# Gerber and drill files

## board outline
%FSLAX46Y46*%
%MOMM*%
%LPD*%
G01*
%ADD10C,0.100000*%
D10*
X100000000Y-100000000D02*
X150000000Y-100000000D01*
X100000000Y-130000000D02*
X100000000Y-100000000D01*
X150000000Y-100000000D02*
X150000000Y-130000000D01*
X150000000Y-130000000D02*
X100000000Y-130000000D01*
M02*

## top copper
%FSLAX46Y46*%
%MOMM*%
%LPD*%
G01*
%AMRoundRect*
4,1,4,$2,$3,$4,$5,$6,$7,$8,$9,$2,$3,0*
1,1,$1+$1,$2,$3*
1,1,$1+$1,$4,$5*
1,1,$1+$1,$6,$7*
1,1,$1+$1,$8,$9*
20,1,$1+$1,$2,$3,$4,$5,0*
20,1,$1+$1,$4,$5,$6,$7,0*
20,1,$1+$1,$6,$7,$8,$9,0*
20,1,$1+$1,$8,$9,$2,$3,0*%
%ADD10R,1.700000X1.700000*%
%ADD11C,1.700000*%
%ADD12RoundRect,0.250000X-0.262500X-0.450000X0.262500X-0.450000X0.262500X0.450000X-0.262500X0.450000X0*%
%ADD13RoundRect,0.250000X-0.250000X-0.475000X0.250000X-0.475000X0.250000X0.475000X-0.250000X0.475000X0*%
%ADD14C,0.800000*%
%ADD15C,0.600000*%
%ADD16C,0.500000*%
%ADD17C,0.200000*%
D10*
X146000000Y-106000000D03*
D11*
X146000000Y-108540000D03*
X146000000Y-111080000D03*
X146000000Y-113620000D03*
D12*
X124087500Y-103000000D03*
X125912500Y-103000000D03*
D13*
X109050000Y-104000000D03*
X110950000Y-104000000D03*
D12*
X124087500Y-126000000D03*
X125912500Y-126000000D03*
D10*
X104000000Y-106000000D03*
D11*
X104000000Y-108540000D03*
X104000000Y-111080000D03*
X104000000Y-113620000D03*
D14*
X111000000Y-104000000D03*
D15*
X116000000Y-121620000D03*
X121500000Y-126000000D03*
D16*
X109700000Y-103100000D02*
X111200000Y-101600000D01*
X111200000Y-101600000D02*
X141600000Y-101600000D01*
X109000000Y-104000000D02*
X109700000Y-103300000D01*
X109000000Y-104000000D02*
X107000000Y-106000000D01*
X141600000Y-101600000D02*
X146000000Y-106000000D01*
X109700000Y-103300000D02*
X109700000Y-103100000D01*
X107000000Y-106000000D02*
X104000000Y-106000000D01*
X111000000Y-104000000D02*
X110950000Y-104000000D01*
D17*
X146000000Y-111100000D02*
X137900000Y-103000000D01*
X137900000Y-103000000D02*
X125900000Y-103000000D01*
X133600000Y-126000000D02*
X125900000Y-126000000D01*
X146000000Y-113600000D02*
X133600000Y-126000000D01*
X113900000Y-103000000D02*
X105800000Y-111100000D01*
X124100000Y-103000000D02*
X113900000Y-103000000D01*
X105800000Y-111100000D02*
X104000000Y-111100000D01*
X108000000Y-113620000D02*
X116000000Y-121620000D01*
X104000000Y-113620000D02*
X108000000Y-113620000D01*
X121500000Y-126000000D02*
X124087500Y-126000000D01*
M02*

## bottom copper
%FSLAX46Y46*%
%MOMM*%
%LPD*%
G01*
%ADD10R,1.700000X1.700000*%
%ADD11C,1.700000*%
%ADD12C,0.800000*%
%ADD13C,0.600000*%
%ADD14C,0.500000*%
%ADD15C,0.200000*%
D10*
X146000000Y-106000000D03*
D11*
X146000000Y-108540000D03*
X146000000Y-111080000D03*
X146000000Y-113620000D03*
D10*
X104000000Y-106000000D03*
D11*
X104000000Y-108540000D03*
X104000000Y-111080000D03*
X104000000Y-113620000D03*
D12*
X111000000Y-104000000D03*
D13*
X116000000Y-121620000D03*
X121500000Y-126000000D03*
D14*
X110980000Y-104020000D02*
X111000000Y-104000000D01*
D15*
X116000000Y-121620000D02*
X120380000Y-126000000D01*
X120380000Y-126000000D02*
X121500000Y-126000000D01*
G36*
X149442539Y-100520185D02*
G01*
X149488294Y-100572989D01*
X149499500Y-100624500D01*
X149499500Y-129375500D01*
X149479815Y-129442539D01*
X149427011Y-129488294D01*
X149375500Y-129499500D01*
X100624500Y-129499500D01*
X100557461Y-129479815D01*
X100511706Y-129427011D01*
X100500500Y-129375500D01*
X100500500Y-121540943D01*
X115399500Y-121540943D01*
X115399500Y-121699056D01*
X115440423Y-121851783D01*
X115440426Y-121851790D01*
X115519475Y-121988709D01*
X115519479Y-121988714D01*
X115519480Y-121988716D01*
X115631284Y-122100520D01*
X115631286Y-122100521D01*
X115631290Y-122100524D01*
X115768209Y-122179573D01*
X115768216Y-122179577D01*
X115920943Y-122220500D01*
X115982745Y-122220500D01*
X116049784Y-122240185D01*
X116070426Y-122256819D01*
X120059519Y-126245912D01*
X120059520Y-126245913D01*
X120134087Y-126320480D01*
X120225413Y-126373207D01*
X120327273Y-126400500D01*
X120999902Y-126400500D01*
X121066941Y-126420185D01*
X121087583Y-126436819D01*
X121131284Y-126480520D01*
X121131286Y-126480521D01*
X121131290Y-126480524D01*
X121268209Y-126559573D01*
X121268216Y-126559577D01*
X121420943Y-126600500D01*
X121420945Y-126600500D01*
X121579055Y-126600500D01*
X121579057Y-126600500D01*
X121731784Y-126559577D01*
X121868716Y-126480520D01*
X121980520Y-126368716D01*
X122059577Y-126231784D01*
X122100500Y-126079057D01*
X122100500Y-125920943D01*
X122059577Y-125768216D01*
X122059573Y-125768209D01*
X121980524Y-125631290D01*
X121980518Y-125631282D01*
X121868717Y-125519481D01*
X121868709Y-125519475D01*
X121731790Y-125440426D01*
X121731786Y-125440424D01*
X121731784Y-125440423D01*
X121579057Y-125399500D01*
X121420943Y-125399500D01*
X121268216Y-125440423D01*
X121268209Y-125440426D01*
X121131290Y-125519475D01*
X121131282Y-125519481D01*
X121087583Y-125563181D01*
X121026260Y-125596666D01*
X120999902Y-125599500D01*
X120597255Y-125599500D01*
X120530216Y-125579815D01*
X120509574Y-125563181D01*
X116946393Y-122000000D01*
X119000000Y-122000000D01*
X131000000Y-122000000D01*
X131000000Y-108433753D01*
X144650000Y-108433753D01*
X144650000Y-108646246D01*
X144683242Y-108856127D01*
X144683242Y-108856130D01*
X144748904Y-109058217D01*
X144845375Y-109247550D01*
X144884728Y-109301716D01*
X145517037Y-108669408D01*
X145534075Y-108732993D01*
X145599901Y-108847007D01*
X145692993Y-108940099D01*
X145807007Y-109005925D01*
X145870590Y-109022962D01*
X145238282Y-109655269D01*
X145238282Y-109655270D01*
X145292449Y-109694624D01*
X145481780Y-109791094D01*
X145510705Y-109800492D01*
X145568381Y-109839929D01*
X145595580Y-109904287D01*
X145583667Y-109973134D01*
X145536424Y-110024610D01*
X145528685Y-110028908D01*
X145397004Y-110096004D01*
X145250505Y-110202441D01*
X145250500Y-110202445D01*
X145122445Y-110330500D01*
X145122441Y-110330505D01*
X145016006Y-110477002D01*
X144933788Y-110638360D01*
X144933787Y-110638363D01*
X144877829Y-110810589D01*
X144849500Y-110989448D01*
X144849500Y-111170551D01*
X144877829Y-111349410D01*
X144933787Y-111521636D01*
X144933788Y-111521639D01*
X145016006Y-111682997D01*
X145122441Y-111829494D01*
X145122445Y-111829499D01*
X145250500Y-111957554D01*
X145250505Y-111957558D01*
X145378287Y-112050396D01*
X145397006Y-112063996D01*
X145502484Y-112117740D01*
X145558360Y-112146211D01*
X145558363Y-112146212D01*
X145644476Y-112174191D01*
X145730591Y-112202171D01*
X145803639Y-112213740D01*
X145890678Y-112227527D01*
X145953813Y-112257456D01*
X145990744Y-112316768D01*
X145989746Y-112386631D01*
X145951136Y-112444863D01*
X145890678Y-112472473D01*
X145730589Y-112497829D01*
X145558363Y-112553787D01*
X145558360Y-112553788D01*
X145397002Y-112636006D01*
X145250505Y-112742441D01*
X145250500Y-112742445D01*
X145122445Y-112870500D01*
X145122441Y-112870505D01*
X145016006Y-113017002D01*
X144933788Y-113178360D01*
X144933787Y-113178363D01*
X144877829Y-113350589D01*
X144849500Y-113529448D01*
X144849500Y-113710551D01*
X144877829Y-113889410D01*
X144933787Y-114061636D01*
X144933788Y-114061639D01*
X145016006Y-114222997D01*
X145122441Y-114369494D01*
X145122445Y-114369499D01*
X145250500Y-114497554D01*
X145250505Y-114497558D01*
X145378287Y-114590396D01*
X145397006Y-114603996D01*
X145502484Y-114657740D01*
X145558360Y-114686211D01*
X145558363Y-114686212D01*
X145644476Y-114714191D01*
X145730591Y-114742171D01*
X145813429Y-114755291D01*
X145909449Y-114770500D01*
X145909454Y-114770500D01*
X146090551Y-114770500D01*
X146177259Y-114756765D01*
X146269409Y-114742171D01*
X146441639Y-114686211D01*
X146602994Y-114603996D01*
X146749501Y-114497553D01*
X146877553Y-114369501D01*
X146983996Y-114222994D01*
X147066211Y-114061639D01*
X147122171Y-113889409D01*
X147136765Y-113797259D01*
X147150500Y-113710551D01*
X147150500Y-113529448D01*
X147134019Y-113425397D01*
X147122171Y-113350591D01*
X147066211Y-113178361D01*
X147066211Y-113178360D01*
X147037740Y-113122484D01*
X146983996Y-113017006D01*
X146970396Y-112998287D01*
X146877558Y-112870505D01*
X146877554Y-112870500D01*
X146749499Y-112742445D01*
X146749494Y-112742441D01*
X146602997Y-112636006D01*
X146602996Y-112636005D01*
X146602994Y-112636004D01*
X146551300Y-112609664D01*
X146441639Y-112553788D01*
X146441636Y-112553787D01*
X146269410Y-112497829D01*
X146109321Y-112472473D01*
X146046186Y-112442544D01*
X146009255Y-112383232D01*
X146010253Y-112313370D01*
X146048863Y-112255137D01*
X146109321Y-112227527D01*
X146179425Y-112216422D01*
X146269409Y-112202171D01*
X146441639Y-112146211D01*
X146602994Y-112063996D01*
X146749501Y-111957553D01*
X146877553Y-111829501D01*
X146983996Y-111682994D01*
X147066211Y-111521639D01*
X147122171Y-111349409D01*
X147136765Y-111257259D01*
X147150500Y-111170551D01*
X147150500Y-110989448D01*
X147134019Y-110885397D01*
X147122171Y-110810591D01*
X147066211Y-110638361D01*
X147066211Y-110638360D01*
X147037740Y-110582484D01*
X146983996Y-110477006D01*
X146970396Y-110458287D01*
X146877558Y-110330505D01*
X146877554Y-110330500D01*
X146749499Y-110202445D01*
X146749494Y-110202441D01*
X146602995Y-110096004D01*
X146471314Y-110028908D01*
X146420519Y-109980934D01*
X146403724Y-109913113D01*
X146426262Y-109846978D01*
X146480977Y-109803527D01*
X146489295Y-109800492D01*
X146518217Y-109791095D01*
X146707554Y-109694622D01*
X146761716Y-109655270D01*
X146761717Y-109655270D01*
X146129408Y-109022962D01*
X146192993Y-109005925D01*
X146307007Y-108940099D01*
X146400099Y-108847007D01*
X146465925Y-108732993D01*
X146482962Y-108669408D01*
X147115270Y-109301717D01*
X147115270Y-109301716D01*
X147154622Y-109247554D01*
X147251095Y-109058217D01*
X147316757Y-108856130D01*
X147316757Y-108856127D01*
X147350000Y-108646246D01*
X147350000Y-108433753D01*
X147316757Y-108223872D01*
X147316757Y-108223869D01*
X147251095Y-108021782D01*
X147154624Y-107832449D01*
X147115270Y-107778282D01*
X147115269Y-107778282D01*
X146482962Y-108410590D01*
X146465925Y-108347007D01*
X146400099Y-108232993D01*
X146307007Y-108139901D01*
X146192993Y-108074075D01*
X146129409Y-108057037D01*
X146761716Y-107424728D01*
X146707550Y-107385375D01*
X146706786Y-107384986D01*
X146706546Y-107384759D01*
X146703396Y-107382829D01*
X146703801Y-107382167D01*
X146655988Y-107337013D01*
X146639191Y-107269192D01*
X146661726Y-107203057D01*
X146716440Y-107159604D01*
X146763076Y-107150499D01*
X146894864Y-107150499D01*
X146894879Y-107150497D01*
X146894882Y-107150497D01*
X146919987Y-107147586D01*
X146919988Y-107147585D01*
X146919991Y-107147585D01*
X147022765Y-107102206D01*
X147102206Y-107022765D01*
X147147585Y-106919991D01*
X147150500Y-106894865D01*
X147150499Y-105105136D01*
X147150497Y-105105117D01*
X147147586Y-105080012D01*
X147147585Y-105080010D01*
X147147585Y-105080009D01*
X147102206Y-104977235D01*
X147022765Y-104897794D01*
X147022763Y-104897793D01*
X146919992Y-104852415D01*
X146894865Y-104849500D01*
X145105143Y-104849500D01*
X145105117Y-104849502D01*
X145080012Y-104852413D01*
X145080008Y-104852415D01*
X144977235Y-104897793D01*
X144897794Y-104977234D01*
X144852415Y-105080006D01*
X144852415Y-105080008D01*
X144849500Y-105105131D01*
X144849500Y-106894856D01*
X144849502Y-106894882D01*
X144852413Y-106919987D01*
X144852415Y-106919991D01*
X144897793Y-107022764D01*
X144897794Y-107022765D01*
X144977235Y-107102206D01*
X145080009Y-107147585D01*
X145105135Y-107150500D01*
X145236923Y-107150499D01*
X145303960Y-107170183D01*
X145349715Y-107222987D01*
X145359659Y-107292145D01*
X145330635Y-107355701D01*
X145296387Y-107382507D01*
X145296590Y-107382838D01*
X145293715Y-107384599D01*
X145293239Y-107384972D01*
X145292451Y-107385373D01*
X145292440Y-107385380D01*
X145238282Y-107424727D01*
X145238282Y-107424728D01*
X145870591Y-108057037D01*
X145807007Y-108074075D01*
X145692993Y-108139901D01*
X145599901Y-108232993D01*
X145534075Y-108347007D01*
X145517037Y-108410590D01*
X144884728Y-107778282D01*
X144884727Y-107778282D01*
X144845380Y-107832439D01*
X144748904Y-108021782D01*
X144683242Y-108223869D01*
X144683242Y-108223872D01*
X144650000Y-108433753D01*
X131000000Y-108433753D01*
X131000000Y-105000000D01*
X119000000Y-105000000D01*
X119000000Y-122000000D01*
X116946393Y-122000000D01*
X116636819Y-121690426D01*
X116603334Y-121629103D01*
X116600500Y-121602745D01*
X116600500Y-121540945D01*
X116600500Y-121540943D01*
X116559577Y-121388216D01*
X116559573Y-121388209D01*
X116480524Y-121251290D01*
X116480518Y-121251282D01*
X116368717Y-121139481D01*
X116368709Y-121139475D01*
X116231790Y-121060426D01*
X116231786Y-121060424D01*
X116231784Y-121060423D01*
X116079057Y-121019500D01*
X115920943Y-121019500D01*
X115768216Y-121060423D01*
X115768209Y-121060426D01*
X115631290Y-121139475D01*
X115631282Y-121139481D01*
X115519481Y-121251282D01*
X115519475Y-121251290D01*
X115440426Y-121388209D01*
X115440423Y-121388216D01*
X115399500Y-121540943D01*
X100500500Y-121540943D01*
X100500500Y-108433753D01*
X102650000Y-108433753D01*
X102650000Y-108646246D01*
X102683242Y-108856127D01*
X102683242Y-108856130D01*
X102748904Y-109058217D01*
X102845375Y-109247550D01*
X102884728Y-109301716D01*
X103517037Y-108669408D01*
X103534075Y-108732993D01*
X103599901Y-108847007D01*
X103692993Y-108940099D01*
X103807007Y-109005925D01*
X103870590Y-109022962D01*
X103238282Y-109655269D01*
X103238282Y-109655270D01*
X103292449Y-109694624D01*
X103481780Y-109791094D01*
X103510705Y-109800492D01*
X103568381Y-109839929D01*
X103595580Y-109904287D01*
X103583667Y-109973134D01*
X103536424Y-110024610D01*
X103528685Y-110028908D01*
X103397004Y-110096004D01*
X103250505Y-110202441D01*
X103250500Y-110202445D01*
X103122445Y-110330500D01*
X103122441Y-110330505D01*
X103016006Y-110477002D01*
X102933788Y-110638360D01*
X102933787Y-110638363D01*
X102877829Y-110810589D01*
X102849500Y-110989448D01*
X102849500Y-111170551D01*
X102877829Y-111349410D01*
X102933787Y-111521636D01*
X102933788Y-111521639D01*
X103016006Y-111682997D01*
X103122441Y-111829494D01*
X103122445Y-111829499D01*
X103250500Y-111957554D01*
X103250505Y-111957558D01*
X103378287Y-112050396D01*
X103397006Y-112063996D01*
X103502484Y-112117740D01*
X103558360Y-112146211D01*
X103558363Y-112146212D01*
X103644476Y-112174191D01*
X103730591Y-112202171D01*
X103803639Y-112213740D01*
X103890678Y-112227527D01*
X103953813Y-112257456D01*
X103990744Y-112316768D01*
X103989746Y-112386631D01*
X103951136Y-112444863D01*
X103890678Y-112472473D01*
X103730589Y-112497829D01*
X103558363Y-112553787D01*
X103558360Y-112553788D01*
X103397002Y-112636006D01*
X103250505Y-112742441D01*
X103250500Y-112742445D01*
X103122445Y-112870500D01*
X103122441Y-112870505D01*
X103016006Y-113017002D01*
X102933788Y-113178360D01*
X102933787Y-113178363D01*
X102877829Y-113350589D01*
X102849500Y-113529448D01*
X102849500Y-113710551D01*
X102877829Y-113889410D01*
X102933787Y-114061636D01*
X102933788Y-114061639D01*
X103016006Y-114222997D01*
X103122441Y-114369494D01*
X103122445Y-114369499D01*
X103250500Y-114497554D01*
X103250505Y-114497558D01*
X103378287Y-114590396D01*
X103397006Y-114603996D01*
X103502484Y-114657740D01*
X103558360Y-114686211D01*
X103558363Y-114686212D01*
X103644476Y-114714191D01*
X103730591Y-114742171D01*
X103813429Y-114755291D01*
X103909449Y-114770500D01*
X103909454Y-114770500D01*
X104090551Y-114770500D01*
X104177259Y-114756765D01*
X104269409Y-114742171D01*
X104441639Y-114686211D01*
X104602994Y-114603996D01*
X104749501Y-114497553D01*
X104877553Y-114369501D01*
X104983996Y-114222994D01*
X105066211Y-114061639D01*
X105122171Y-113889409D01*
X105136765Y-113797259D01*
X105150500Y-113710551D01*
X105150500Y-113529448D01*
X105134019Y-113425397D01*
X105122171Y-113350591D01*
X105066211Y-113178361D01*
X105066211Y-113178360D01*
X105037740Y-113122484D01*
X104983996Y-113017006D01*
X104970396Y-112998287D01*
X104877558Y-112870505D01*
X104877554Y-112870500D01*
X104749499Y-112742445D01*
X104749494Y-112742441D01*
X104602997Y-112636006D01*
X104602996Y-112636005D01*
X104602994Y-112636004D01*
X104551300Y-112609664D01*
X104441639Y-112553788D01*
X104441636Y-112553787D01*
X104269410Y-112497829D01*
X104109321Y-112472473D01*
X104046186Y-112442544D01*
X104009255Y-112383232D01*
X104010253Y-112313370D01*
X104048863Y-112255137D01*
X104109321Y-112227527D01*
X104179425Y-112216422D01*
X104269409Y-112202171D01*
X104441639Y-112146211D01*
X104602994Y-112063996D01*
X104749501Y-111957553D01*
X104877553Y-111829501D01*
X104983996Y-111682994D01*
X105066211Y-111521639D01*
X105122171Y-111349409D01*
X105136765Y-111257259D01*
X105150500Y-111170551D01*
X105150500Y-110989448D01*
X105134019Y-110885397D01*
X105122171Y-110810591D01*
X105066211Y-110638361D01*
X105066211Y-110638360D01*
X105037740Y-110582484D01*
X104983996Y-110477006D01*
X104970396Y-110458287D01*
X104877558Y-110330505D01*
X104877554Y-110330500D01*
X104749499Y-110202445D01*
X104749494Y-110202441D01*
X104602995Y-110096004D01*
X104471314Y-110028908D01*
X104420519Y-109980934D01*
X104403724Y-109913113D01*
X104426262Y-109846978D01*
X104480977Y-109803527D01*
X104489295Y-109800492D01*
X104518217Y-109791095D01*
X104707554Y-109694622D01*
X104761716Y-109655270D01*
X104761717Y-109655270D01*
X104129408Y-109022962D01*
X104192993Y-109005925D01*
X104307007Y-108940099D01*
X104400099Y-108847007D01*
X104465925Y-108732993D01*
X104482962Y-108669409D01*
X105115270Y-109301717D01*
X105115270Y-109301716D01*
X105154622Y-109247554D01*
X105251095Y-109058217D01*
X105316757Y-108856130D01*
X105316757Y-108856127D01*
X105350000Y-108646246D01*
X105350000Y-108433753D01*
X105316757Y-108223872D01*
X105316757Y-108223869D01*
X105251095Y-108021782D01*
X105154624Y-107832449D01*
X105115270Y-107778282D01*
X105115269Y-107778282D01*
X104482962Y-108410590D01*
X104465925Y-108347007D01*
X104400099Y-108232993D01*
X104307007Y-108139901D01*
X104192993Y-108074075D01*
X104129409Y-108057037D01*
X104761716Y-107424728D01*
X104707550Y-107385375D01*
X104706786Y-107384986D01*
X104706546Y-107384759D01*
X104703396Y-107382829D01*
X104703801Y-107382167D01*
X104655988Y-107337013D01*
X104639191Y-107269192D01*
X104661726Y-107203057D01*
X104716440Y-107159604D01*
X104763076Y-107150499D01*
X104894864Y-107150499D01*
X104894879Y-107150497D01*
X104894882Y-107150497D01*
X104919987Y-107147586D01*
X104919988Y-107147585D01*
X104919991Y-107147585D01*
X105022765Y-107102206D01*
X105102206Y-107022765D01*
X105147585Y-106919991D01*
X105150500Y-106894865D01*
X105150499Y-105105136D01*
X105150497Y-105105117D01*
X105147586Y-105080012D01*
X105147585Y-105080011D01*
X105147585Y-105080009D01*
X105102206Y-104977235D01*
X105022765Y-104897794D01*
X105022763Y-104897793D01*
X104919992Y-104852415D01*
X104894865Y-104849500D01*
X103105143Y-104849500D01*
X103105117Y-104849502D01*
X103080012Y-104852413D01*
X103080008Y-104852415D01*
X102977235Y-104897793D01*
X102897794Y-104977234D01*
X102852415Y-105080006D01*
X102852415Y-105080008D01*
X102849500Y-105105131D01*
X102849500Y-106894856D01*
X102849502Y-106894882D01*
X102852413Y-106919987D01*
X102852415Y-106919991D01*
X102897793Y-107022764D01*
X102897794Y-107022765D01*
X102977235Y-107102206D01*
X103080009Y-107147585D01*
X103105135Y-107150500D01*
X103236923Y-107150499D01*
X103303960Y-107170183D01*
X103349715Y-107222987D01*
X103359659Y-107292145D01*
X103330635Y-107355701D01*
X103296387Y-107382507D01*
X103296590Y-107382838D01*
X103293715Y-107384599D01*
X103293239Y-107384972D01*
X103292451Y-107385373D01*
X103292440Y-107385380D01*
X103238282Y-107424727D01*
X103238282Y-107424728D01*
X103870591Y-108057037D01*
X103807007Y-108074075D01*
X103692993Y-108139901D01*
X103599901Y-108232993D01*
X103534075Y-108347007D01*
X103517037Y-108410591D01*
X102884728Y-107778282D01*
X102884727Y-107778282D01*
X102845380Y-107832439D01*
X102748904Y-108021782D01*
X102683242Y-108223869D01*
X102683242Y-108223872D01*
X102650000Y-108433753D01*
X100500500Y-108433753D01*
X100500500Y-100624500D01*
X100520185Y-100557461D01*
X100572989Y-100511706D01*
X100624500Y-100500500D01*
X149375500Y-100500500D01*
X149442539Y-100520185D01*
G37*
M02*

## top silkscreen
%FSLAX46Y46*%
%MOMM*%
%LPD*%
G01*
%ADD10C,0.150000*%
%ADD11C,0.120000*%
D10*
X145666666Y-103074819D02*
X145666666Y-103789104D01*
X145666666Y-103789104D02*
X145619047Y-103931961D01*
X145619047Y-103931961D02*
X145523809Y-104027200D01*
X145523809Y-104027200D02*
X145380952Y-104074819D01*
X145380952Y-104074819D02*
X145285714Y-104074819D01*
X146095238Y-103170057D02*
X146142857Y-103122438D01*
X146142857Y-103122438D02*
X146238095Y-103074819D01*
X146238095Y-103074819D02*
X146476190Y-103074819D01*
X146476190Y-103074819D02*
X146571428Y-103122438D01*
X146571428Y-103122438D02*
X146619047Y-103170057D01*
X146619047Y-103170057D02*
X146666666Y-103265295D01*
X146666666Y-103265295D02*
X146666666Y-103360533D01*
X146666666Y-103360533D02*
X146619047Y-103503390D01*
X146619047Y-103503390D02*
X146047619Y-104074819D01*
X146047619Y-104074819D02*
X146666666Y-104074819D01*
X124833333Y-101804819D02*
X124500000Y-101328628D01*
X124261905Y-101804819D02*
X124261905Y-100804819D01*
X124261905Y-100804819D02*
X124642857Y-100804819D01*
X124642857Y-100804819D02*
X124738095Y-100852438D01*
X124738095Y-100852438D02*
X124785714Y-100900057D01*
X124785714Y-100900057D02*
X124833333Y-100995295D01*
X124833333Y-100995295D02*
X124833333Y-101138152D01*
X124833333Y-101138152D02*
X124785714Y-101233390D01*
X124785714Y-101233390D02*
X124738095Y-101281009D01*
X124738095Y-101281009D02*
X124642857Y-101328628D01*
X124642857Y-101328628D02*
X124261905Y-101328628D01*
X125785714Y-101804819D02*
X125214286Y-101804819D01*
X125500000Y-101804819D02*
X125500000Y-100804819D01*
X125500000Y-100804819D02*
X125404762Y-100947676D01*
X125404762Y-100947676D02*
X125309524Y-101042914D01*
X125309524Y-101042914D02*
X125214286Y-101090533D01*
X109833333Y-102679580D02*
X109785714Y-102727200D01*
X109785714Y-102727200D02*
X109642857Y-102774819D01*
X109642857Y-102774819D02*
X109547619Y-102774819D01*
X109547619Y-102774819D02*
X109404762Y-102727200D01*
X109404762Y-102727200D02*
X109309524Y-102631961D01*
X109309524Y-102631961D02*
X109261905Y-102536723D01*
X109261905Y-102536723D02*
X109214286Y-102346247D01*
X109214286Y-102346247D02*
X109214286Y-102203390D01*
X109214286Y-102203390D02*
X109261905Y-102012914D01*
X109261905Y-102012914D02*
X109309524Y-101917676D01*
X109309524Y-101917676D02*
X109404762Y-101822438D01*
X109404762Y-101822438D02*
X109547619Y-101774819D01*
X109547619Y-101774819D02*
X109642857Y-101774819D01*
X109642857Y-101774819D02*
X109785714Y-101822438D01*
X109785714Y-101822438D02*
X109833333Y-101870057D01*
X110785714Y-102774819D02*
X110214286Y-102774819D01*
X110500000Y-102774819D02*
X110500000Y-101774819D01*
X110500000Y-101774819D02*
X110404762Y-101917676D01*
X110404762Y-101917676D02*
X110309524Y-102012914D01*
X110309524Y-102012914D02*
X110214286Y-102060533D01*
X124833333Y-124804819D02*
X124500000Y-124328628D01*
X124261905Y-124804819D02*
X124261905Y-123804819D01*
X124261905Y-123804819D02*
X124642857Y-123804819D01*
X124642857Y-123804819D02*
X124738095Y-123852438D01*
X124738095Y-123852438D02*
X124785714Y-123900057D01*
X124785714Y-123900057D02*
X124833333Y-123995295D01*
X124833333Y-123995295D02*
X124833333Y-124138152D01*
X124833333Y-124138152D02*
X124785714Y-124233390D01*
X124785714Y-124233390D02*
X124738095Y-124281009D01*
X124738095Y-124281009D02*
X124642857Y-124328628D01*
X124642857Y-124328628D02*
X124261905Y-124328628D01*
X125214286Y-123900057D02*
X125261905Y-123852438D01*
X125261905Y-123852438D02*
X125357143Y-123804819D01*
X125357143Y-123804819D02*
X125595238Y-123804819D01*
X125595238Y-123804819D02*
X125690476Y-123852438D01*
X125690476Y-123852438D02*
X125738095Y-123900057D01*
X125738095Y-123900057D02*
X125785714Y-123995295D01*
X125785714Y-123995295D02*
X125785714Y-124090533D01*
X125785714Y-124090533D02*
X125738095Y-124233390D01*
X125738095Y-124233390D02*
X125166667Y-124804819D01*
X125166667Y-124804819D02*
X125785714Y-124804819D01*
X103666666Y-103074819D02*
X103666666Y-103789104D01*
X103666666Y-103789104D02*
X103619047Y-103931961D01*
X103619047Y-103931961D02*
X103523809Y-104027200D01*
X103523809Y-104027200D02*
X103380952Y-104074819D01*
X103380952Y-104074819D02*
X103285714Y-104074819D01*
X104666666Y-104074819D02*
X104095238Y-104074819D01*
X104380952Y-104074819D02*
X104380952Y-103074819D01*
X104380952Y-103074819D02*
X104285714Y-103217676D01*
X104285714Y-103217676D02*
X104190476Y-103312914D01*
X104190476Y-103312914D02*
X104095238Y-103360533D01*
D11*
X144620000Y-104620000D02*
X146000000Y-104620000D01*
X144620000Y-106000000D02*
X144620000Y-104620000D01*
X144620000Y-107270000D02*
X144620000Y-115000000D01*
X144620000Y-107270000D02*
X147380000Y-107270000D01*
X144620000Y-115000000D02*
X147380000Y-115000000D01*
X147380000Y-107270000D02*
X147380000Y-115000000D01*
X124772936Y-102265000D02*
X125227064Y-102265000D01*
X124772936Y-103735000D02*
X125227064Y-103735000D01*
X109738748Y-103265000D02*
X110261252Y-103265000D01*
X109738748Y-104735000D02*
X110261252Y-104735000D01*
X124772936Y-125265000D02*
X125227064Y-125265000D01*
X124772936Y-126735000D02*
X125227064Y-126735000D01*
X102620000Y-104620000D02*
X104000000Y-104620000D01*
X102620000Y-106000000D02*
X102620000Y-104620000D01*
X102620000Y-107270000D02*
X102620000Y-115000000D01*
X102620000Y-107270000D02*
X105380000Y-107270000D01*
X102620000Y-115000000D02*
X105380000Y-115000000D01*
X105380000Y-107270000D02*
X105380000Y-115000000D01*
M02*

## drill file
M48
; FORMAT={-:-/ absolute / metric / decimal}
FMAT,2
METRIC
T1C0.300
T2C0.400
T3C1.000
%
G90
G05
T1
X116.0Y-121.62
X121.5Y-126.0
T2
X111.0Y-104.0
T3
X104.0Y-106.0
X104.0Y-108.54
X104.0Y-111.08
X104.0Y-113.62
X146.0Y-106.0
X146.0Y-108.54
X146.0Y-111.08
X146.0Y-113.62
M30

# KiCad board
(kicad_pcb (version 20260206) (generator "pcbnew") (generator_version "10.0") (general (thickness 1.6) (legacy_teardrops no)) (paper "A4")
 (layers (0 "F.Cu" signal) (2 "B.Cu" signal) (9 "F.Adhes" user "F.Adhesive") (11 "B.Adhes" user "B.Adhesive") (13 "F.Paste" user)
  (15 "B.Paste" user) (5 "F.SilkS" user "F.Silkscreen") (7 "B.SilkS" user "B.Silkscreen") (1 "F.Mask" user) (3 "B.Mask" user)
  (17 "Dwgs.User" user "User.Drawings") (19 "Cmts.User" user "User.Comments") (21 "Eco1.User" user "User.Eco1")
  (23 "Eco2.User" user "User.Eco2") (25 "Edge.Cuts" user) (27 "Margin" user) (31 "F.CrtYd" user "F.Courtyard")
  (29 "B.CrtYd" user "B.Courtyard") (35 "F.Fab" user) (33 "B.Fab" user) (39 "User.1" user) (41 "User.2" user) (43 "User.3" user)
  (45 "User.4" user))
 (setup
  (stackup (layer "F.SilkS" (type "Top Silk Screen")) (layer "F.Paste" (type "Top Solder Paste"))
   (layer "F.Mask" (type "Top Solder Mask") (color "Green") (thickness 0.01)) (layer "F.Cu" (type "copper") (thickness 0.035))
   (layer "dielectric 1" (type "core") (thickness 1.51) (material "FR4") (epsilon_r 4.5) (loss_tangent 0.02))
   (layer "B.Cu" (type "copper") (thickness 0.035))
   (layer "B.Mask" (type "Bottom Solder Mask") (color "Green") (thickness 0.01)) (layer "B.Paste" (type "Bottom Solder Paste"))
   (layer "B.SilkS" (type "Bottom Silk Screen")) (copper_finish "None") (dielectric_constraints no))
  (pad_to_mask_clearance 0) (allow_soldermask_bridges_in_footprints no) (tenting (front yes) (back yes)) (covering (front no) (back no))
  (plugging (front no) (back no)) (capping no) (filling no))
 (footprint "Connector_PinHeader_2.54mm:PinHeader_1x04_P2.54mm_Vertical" (layer "F.Cu") (at 146 106)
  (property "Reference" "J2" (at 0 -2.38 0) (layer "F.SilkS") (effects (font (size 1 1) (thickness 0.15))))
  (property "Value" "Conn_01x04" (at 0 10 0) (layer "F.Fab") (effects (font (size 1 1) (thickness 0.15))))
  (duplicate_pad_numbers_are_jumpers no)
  (fp_line (start -1.38 -1.38) (end 0 -1.38) (stroke (width 0.12) (type solid)) (layer "F.SilkS"))
  (fp_line (start -1.38 0) (end -1.38 -1.38) (stroke (width 0.12) (type solid)) (layer "F.SilkS"))
  (fp_line (start -1.38 1.27) (end -1.38 9) (stroke (width 0.12) (type solid)) (layer "F.SilkS"))
  (fp_line (start -1.38 1.27) (end 1.38 1.27) (stroke (width 0.12) (type solid)) (layer "F.SilkS"))
  (fp_line (start -1.38 9) (end 1.38 9) (stroke (width 0.12) (type solid)) (layer "F.SilkS"))
  (fp_line (start 1.38 1.27) (end 1.38 9) (stroke (width 0.12) (type solid)) (layer "F.SilkS"))
  (pad "1" thru_hole rect (at 0 0) (size 1.7 1.7) (drill 1) (layers "*.Cu" "*.Mask") (remove_unused_layers no) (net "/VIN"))
  (pad "2" thru_hole circle (at 0 2.54) (size 1.7 1.7) (drill 1) (layers "*.Cu" "*.Mask") (remove_unused_layers no) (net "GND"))
  (pad "3" thru_hole circle (at 0 5.08) (size 1.7 1.7) (drill 1) (layers "*.Cu" "*.Mask") (remove_unused_layers no) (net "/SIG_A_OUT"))
  (pad "4" thru_hole circle (at 0 7.62) (size 1.7 1.7) (drill 1) (layers "*.Cu" "*.Mask") (remove_unused_layers no) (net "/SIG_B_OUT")))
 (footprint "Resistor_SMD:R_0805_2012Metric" (layer "F.Cu") (at 125 103)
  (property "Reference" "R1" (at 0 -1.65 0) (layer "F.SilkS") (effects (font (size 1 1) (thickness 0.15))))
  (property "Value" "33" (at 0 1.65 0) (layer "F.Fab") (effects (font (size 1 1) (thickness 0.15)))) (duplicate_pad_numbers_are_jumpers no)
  (fp_line (start -0.227064 -0.735) (end 0.227064 -0.735) (stroke (width 0.12) (type solid)) (layer "F.SilkS"))
  (fp_line (start -0.227064 0.735) (end 0.227064 0.735) (stroke (width 0.12) (type solid)) (layer "F.SilkS"))
  (pad "1" smd roundrect (at -0.9125 0) (size 1.025 1.4) (layers "F.Cu" "F.Mask" "F.Paste") (roundrect_rratio 0.243902) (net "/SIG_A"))
  (pad "2" smd roundrect (at 0.9125 0) (size 1.025 1.4) (layers "F.Cu" "F.Mask" "F.Paste") (roundrect_rratio 0.243902) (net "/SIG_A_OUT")))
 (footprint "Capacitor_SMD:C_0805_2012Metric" (layer "F.Cu") (at 110 104)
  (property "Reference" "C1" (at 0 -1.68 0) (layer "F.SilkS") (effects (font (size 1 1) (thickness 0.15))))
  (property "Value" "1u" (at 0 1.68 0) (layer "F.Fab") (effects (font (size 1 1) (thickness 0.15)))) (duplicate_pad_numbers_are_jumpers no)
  (fp_line (start -0.261252 -0.735) (end 0.261252 -0.735) (stroke (width 0.12) (type solid)) (layer "F.SilkS"))
  (fp_line (start -0.261252 0.735) (end 0.261252 0.735) (stroke (width 0.12) (type solid)) (layer "F.SilkS"))
  (pad "1" smd roundrect (at -0.95 0) (size 1 1.45) (layers "F.Cu" "F.Mask" "F.Paste") (roundrect_rratio 0.25) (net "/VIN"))
  (pad "2" smd roundrect (at 0.95 0) (size 1 1.45) (layers "F.Cu" "F.Mask" "F.Paste") (roundrect_rratio 0.25) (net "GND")))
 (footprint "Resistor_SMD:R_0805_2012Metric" (layer "F.Cu") (at 125 126)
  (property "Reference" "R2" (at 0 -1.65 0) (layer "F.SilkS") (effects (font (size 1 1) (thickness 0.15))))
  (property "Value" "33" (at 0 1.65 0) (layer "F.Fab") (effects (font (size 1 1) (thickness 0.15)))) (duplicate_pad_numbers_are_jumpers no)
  (fp_line (start -0.227064 -0.735) (end 0.227064 -0.735) (stroke (width 0.12) (type solid)) (layer "F.SilkS"))
  (fp_line (start -0.227064 0.735) (end 0.227064 0.735) (stroke (width 0.12) (type solid)) (layer "F.SilkS"))
  (pad "1" smd roundrect (at -0.9125 0) (size 1.025 1.4) (layers "F.Cu" "F.Mask" "F.Paste") (roundrect_rratio 0.243902) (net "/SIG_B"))
  (pad "2" smd roundrect (at 0.9125 0) (size 1.025 1.4) (layers "F.Cu" "F.Mask" "F.Paste") (roundrect_rratio 0.243902) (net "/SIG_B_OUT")))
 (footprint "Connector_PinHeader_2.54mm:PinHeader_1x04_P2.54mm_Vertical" (layer "F.Cu") (at 104 106)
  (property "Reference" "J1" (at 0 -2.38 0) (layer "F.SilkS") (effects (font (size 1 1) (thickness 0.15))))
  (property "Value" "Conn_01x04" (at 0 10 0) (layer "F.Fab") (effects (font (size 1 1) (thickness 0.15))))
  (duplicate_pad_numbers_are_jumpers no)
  (fp_line (start -1.38 -1.38) (end 0 -1.38) (stroke (width 0.12) (type solid)) (layer "F.SilkS"))
  (fp_line (start -1.38 0) (end -1.38 -1.38) (stroke (width 0.12) (type solid)) (layer "F.SilkS"))
  (fp_line (start -1.38 1.27) (end -1.38 9) (stroke (width 0.12) (type solid)) (layer "F.SilkS"))
  (fp_line (start -1.38 1.27) (end 1.38 1.27) (stroke (width 0.12) (type solid)) (layer "F.SilkS"))
  (fp_line (start -1.38 9) (end 1.38 9) (stroke (width 0.12) (type solid)) (layer "F.SilkS"))
  (fp_line (start 1.38 1.27) (end 1.38 9) (stroke (width 0.12) (type solid)) (layer "F.SilkS"))
  (pad "1" thru_hole rect (at 0 0) (size 1.7 1.7) (drill 1) (layers "*.Cu" "*.Mask") (remove_unused_layers no) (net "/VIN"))
  (pad "2" thru_hole circle (at 0 2.54) (size 1.7 1.7) (drill 1) (layers "*.Cu" "*.Mask") (remove_unused_layers no) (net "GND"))
  (pad "3" thru_hole circle (at 0 5.08) (size 1.7 1.7) (drill 1) (layers "*.Cu" "*.Mask") (remove_unused_layers no) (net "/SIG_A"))
  (pad "4" thru_hole circle (at 0 7.62) (size 1.7 1.7) (drill 1) (layers "*.Cu" "*.Mask") (remove_unused_layers no) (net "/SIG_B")))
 (gr_line (start 100 100) (end 150 100) (stroke (width 0.1) (type default)) (layer "Edge.Cuts"))
 (gr_line (start 100 130) (end 100 100) (stroke (width 0.1) (type default)) (layer "Edge.Cuts"))
 (gr_line (start 150 100) (end 150 130) (stroke (width 0.1) (type default)) (layer "Edge.Cuts"))
 (gr_line (start 150 130) (end 100 130) (stroke (width 0.1) (type default)) (layer "Edge.Cuts"))
 (segment (start 109.7 103.1) (end 111.2 101.6) (width 0.5) (layer "F.Cu") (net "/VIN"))
 (segment (start 111.2 101.6) (end 141.6 101.6) (width 0.5) (layer "F.Cu") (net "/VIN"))
 (segment (start 109 104) (end 109.7 103.3) (width 0.5) (layer "F.Cu") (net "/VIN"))
 (segment (start 109 104) (end 107 106) (width 0.5) (layer "F.Cu") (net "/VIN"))
 (segment (start 141.6 101.6) (end 146 106) (width 0.5) (layer "F.Cu") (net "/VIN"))
 (segment (start 109.7 103.3) (end 109.7 103.1) (width 0.5) (layer "F.Cu") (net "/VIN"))
 (segment (start 107 106) (end 104 106) (width 0.5) (layer "F.Cu") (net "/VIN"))
 (segment (start 111 104) (end 110.95 104) (width 0.5) (layer "F.Cu") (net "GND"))
 (via (at 111 104) (size 0.8) (drill 0.4) (layers "F.Cu" "B.Cu") (capping yes) (filling yes) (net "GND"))
 (segment (start 110.98 104.02) (end 111 104) (width 0.5) (layer "B.Cu") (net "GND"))
 (segment (start 146 111.1) (end 137.9 103) (width 0.2) (layer "F.Cu") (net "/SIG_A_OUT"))
 (segment (start 137.9 103) (end 125.9 103) (width 0.2) (layer "F.Cu") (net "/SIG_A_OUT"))
 (segment (start 133.6 126) (end 125.9 126) (width 0.2) (layer "F.Cu") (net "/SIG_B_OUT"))
 (segment (start 146 113.6) (end 133.6 126) (width 0.2) (layer "F.Cu") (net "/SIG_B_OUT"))
 (segment (start 113.9 103) (end 105.8 111.1) (width 0.2) (layer "F.Cu") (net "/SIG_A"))
 (segment (start 124.1 103) (end 113.9 103) (width 0.2) (layer "F.Cu") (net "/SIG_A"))
 (segment (start 105.8 111.1) (end 104 111.1) (width 0.2) (layer "F.Cu") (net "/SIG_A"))
 (segment (start 108 113.62) (end 116 121.62) (width 0.2) (locked yes) (layer "F.Cu") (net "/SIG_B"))
 (segment (start 104 113.62) (end 108 113.62) (width 0.2) (locked yes) (layer "F.Cu") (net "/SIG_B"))
 (segment (start 121.5 126) (end 124.0875 126) (width 0.2) (locked yes) (layer "F.Cu") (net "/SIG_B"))
 (via (at 116 121.62) (size 0.6) (drill 0.3) (layers "F.Cu" "B.Cu") (locked yes) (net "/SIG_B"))
 (via (at 121.5 126) (size 0.6) (drill 0.3) (layers "F.Cu" "B.Cu") (locked yes) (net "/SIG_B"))
 (segment (start 116 121.62) (end 120.38 126) (width 0.2) (locked yes) (layer "B.Cu") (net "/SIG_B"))
 (segment (start 120.38 126) (end 121.5 126) (width 0.2) (locked yes) (layer "B.Cu") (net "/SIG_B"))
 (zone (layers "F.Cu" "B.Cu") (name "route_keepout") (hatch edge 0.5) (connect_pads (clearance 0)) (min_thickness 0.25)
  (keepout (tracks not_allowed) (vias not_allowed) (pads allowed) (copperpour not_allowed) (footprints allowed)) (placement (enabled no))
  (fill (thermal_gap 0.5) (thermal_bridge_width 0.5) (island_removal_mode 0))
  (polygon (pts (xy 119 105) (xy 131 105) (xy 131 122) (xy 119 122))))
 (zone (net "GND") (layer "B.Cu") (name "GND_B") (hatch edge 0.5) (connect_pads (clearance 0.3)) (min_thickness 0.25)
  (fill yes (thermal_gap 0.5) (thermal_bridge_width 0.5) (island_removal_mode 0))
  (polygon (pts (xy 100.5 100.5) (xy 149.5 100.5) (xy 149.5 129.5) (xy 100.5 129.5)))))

